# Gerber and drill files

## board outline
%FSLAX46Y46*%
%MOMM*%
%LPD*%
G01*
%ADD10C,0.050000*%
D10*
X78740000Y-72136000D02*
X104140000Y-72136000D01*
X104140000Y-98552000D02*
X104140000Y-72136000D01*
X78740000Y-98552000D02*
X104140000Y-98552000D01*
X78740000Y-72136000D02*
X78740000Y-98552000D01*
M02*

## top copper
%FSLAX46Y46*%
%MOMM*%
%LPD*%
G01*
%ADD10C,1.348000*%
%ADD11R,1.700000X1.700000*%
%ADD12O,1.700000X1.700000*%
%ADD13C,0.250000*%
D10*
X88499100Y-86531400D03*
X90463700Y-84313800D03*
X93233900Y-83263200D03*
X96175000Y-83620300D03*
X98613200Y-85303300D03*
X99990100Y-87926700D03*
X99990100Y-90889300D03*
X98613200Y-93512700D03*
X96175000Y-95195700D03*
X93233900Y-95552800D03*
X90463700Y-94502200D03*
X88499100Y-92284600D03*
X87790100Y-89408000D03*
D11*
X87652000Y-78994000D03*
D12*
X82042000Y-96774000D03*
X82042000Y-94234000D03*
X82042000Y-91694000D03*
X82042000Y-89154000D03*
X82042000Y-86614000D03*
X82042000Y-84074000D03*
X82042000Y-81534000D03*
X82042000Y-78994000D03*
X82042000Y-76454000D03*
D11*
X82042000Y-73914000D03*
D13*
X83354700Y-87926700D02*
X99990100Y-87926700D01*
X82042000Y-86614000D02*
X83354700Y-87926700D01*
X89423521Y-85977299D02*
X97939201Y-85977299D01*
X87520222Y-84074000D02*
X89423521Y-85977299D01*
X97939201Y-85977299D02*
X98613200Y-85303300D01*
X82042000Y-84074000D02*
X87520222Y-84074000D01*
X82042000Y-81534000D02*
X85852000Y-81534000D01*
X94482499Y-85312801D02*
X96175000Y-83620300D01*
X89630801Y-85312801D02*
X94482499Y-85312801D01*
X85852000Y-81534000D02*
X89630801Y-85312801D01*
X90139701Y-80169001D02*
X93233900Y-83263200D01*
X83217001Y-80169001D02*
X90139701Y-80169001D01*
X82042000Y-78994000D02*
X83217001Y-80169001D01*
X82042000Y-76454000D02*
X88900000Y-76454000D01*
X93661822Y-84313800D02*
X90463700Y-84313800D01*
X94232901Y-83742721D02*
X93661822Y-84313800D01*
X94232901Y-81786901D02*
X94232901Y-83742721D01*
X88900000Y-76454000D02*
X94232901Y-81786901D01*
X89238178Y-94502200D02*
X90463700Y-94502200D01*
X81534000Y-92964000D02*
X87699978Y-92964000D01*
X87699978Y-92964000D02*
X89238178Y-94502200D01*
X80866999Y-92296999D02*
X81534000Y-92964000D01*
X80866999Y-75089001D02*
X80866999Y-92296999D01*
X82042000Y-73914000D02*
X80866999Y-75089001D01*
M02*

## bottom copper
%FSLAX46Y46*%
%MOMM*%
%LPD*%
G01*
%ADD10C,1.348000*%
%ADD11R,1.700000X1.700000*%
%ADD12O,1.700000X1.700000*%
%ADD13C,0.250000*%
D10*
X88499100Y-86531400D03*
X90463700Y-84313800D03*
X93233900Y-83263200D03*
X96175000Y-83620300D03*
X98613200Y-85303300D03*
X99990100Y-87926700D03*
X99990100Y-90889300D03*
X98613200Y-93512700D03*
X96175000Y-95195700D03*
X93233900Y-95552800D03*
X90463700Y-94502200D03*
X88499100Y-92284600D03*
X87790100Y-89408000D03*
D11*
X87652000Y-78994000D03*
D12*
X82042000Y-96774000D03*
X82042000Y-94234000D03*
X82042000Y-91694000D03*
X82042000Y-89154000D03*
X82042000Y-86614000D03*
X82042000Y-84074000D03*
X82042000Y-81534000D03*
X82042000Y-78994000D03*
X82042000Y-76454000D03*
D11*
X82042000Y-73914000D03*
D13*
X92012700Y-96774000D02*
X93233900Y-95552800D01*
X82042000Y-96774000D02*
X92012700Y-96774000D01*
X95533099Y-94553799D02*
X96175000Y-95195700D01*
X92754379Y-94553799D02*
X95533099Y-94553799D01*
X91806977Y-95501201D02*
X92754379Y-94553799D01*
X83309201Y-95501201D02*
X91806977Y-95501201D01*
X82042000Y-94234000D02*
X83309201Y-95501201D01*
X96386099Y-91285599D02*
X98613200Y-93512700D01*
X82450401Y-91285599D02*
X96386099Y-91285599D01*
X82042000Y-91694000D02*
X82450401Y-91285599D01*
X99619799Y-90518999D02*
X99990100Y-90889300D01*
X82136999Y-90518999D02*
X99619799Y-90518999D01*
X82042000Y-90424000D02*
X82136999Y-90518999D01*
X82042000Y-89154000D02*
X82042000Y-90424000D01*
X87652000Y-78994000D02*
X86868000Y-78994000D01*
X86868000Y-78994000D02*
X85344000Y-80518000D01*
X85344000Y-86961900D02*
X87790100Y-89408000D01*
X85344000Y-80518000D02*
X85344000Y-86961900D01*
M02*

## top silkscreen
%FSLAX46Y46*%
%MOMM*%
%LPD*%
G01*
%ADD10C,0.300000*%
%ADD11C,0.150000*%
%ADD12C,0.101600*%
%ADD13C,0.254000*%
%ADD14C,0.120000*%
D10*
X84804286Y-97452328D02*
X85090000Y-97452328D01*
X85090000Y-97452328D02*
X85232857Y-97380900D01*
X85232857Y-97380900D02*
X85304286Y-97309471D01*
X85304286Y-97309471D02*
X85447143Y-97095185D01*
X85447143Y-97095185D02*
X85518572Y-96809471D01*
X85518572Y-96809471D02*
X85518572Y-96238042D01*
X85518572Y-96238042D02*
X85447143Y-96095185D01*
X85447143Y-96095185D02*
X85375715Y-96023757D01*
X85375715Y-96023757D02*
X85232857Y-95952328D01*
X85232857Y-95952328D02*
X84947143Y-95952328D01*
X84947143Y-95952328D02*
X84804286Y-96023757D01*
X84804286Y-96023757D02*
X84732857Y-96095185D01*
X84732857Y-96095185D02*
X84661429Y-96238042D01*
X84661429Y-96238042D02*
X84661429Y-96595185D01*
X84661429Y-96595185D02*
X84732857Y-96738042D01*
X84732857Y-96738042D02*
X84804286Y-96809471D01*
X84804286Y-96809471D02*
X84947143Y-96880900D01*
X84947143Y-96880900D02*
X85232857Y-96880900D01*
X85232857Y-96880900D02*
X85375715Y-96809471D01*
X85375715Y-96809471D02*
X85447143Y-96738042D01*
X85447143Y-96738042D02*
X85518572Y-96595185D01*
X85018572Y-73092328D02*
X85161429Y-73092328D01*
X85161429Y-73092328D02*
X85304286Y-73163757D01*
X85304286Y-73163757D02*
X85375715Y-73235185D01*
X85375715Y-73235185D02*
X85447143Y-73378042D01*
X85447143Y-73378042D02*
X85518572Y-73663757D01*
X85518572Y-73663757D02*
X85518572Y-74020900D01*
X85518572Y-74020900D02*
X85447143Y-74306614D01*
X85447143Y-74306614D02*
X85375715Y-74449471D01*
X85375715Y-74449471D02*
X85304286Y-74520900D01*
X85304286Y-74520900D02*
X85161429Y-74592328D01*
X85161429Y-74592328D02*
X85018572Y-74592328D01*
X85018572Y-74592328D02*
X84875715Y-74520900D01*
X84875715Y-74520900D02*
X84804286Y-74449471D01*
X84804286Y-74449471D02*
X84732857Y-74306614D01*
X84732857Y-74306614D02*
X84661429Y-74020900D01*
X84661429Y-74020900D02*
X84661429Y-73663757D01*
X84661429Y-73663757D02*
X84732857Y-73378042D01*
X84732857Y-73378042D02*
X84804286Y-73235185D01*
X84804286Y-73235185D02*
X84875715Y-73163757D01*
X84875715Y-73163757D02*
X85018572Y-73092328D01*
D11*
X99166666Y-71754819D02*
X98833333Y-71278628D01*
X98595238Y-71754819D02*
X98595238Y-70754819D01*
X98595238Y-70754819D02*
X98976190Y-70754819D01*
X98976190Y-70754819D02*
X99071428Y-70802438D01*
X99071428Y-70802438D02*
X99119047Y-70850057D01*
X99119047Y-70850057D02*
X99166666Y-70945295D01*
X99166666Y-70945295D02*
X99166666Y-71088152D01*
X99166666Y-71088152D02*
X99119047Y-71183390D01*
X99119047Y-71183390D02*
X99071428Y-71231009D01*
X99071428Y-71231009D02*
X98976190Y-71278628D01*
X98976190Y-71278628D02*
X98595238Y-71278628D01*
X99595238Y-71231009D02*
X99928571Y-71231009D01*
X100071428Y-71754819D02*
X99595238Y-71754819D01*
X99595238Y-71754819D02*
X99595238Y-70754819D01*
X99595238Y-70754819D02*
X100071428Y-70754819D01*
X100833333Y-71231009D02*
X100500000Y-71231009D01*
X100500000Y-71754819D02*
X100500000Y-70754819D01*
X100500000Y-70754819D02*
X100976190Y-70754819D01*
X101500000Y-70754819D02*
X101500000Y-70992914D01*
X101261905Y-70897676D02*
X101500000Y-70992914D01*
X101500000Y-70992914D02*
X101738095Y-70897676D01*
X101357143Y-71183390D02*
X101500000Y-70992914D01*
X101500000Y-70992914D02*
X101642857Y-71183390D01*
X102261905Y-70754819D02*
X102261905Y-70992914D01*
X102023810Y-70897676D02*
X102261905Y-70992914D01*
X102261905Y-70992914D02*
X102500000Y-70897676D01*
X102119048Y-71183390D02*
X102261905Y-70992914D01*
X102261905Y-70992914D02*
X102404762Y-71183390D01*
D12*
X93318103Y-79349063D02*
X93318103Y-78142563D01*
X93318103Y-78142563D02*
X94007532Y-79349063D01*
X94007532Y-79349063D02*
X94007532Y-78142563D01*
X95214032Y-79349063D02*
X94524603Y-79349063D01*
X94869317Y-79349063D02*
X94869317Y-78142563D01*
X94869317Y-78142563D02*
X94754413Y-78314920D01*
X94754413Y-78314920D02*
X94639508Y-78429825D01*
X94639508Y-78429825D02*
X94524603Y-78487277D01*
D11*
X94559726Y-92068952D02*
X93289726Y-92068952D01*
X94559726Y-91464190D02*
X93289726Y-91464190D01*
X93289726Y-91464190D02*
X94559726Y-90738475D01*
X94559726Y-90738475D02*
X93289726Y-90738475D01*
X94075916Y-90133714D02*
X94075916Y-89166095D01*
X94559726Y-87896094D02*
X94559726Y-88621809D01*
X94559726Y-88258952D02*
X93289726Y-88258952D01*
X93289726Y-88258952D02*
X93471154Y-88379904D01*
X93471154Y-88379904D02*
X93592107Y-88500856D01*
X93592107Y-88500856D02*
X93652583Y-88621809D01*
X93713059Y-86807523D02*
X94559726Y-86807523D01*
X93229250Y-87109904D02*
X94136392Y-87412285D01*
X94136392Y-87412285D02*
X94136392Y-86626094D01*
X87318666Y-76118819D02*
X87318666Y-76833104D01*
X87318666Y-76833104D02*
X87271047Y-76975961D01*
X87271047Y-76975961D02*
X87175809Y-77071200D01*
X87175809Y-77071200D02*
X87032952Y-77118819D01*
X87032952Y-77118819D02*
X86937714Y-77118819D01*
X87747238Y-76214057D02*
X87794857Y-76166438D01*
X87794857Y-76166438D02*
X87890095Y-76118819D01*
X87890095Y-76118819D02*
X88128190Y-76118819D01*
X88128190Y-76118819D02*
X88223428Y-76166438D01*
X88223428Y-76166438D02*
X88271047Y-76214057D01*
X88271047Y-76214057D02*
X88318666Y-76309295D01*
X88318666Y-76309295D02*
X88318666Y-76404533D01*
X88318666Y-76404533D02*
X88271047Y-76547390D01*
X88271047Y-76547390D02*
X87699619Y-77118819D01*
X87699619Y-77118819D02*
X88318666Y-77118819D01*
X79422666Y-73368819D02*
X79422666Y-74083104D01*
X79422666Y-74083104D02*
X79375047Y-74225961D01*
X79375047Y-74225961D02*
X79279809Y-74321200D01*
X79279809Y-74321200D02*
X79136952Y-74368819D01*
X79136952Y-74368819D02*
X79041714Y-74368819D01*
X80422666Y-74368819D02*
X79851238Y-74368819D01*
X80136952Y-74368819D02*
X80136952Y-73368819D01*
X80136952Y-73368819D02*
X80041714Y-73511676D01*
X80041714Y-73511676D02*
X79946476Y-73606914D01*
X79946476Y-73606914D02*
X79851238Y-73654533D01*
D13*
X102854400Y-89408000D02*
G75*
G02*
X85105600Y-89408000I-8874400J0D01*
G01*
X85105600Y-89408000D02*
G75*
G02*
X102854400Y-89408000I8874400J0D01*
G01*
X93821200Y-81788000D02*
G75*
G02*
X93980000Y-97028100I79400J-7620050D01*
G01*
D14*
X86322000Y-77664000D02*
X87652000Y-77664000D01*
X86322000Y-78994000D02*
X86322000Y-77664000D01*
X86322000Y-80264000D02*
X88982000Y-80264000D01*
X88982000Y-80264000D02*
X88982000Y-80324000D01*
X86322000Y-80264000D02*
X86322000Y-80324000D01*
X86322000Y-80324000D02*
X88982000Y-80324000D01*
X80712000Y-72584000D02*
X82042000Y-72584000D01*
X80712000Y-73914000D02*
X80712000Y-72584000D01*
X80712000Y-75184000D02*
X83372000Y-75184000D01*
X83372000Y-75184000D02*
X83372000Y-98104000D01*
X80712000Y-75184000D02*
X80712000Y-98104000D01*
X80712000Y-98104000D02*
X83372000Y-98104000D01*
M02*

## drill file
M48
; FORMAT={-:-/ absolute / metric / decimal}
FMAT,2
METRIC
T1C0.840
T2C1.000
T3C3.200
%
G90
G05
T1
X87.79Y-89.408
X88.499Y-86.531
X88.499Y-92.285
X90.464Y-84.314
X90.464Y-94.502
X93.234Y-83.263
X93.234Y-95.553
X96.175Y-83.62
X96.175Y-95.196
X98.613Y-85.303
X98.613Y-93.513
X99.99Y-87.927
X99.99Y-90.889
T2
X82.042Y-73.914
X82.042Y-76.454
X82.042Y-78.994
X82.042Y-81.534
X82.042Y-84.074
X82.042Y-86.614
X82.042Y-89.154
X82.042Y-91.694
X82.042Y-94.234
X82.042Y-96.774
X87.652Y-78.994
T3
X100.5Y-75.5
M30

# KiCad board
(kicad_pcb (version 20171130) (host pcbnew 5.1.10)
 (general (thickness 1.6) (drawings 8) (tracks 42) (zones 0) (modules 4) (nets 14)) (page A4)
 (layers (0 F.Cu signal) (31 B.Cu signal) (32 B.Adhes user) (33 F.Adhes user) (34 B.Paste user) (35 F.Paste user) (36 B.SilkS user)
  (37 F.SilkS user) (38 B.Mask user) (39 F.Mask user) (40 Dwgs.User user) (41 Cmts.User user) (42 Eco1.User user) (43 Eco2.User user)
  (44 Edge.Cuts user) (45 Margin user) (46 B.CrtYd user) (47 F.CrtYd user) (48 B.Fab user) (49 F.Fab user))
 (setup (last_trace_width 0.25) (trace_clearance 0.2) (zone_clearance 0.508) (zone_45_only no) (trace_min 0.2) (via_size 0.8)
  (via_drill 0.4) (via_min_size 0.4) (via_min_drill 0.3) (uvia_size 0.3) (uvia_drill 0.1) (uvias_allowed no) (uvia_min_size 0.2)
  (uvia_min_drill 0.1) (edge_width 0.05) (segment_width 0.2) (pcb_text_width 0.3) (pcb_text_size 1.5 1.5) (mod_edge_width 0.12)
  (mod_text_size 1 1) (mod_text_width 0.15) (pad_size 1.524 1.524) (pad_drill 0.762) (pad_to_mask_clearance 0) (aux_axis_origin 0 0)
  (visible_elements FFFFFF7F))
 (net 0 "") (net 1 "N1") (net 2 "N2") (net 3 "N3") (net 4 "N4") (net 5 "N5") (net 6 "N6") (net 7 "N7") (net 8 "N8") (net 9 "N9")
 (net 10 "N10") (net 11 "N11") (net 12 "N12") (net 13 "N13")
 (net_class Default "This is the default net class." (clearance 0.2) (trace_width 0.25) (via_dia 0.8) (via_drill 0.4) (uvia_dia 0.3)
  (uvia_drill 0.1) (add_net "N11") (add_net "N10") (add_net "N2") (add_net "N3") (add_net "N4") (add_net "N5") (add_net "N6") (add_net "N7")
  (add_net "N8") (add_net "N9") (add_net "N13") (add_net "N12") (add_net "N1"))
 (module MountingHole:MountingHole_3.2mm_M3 (layer F.Cu) (at 100.5 75.5)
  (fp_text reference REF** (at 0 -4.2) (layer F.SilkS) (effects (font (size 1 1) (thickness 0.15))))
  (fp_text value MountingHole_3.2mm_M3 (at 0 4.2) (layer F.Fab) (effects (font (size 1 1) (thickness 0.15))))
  (pad 1 np_thru_hole circle (at 0 0) (size 3.2 3.2) (drill 3.2) (layers *.Cu *.Mask)))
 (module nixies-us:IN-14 (layer F.Cu) (at 93.98 89.408 270)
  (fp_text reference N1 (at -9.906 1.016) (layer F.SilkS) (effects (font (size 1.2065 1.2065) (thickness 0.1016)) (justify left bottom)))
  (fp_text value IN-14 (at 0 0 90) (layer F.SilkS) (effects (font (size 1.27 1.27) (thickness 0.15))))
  (fp_circle (center 0 0) (end 8.8744 0) (layer F.SilkS) (width 0.254))
  (fp_arc (start 0.00005 0.0794) (end -7.62 0.1588) (angle 180) (layer F.SilkS) (width 0.254))
  (pad RHDP thru_hole circle (at -2.8766 5.4809 270) (size 1.348 1.348) (drill 0.84) (layers *.Cu *.Mask) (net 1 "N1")
   (solder_mask_margin 0.1016))
  (pad 1 thru_hole circle (at -5.0942 3.5163 270) (size 1.348 1.348) (drill 0.84) (layers *.Cu *.Mask) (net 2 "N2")
   (solder_mask_margin 0.1016))
  (pad 2 thru_hole circle (at -6.1448 0.7461 270) (size 1.348 1.348) (drill 0.84) (layers *.Cu *.Mask) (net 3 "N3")
   (solder_mask_margin 0.1016))
  (pad 3 thru_hole circle (at -5.7877 -2.195 270) (size 1.348 1.348) (drill 0.84) (layers *.Cu *.Mask) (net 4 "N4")
   (solder_mask_margin 0.1016))
  (pad 4 thru_hole circle (at -4.1047 -4.6332 270) (size 1.348 1.348) (drill 0.84) (layers *.Cu *.Mask) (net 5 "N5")
   (solder_mask_margin 0.1016))
  (pad 5 thru_hole circle (at -1.4813 -6.0101 270) (size 1.348 1.348) (drill 0.84) (layers *.Cu *.Mask) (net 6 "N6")
   (solder_mask_margin 0.1016))
  (pad 6 thru_hole circle (at 1.4813 -6.0101 270) (size 1.348 1.348) (drill 0.84) (layers *.Cu *.Mask) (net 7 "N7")
   (solder_mask_margin 0.1016))
  (pad 7 thru_hole circle (at 4.1047 -4.6332 270) (size 1.348 1.348) (drill 0.84) (layers *.Cu *.Mask) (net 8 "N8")
   (solder_mask_margin 0.1016))
  (pad 8 thru_hole circle (at 5.7877 -2.195 270) (size 1.348 1.348) (drill 0.84) (layers *.Cu *.Mask) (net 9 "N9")
   (solder_mask_margin 0.1016))
  (pad 9 thru_hole circle (at 6.1448 0.7461 270) (size 1.348 1.348) (drill 0.84) (layers *.Cu *.Mask) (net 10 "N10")
   (solder_mask_margin 0.1016))
  (pad 0 thru_hole circle (at 5.0942 3.5163 270) (size 1.348 1.348) (drill 0.84) (layers *.Cu *.Mask) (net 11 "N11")
   (solder_mask_margin 0.1016))
  (pad LHDP thru_hole circle (at 2.8766 5.4809 270) (size 1.348 1.348) (drill 0.84) (layers *.Cu *.Mask) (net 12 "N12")
   (solder_mask_margin 0.1016))
  (pad A thru_hole circle (at 0 6.1899 270) (size 1.348 1.348) (drill 0.84) (layers *.Cu *.Mask) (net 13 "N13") (solder_mask_margin 0.1016)))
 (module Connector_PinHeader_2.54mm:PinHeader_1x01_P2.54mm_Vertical (layer F.Cu) (at 87.652 78.994)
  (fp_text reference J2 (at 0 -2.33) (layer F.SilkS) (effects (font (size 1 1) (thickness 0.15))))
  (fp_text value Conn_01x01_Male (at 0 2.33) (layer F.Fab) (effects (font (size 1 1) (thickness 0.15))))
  (fp_line (start -1.33 -1.33) (end 0 -1.33) (layer F.SilkS) (width 0.12))
  (fp_line (start -1.33 0) (end -1.33 -1.33) (layer F.SilkS) (width 0.12))
  (fp_line (start -1.33 1.27) (end 1.33 1.27) (layer F.SilkS) (width 0.12))
  (fp_line (start 1.33 1.27) (end 1.33 1.33) (layer F.SilkS) (width 0.12))
  (fp_line (start -1.33 1.27) (end -1.33 1.33) (layer F.SilkS) (width 0.12))
  (fp_line (start -1.33 1.33) (end 1.33 1.33) (layer F.SilkS) (width 0.12))
  (pad 1 thru_hole rect (at 0 0) (size 1.7 1.7) (drill 1) (layers *.Cu *.Mask) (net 13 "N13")))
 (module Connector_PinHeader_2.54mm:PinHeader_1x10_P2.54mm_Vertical (layer F.Cu) (at 82.042 73.914)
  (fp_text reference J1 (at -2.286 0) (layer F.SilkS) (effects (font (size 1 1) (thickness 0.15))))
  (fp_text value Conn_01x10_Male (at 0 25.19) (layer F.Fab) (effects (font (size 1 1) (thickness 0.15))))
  (fp_line (start -1.33 -1.33) (end 0 -1.33) (layer F.SilkS) (width 0.12))
  (fp_line (start -1.33 0) (end -1.33 -1.33) (layer F.SilkS) (width 0.12))
  (fp_line (start -1.33 1.27) (end 1.33 1.27) (layer F.SilkS) (width 0.12))
  (fp_line (start 1.33 1.27) (end 1.33 24.19) (layer F.SilkS) (width 0.12))
  (fp_line (start -1.33 1.27) (end -1.33 24.19) (layer F.SilkS) (width 0.12))
  (fp_line (start -1.33 24.19) (end 1.33 24.19) (layer F.SilkS) (width 0.12))
  (pad 10 thru_hole oval (at 0 22.86) (size 1.7 1.7) (drill 1) (layers *.Cu *.Mask) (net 10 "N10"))
  (pad 9 thru_hole oval (at 0 20.32) (size 1.7 1.7) (drill 1) (layers *.Cu *.Mask) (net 9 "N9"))
  (pad 8 thru_hole oval (at 0 17.78) (size 1.7 1.7) (drill 1) (layers *.Cu *.Mask) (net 8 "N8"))
  (pad 7 thru_hole oval (at 0 15.24) (size 1.7 1.7) (drill 1) (layers *.Cu *.Mask) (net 7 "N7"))
  (pad 6 thru_hole oval (at 0 12.7) (size 1.7 1.7) (drill 1) (layers *.Cu *.Mask) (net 6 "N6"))
  (pad 5 thru_hole oval (at 0 10.16) (size 1.7 1.7) (drill 1) (layers *.Cu *.Mask) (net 5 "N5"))
  (pad 4 thru_hole oval (at 0 7.62) (size 1.7 1.7) (drill 1) (layers *.Cu *.Mask) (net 4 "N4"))
  (pad 3 thru_hole oval (at 0 5.08) (size 1.7 1.7) (drill 1) (layers *.Cu *.Mask) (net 3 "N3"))
  (pad 2 thru_hole oval (at 0 2.54) (size 1.7 1.7) (drill 1) (layers *.Cu *.Mask) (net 2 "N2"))
  (pad 1 thru_hole rect (at 0 0) (size 1.7 1.7) (drill 1) (layers *.Cu *.Mask) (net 11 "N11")))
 (gr_line (start 78.74 72.136) (end 104.14 72.136) (layer Edge.Cuts) (width 0.05))
 (gr_line (start 104.14 98.552) (end 104.14 72.136) (layer Edge.Cuts) (width 0.05))
 (gr_line (start 78.74 98.552) (end 104.14 98.552) (layer Edge.Cuts) (width 0.05))
 (gr_line (start 78.74 72.136) (end 78.74 98.552) (layer Edge.Cuts) (width 0.05))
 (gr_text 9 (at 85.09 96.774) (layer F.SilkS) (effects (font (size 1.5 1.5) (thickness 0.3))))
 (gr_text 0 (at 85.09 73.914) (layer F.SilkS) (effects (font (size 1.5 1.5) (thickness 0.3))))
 (segment (start 92.0127 96.774) (end 93.2339 95.5528) (width 0.25) (layer B.Cu) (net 10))
 (segment (start 82.042 96.774) (end 92.0127 96.774) (width 0.25) (layer B.Cu) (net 10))
 (segment (start 95.533099 94.553799) (end 96.175 95.1957) (width 0.25) (layer B.Cu) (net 9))
 (segment (start 92.754379 94.553799) (end 95.533099 94.553799) (width 0.25) (layer B.Cu) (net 9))
 (segment (start 91.806977 95.501201) (end 92.754379 94.553799) (width 0.25) (layer B.Cu) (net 9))
 (segment (start 83.309201 95.501201) (end 91.806977 95.501201) (width 0.25) (layer B.Cu) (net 9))
 (segment (start 82.042 94.234) (end 83.309201 95.501201) (width 0.25) (layer B.Cu) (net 9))
 (segment (start 96.386099 91.285599) (end 98.6132 93.5127) (width 0.25) (layer B.Cu) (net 8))
 (segment (start 82.450401 91.285599) (end 96.386099 91.285599) (width 0.25) (layer B.Cu) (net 8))
 (segment (start 82.042 91.694) (end 82.450401 91.285599) (width 0.25) (layer B.Cu) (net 8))
 (segment (start 99.619799 90.518999) (end 99.9901 90.8893) (width 0.25) (layer B.Cu) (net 7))
 (segment (start 82.136999 90.518999) (end 99.619799 90.518999) (width 0.25) (layer B.Cu) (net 7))
 (segment (start 82.042 90.424) (end 82.136999 90.518999) (width 0.25) (layer B.Cu) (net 7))
 (segment (start 82.042 89.154) (end 82.042 90.424) (width 0.25) (layer B.Cu) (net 7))
 (segment (start 83.3547 87.9267) (end 99.9901 87.9267) (width 0.25) (layer F.Cu) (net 6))
 (segment (start 82.042 86.614) (end 83.3547 87.9267) (width 0.25) (layer F.Cu) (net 6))
 (segment (start 89.423521 85.977299) (end 97.939201 85.977299) (width 0.25) (layer F.Cu) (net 5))
 (segment (start 87.520222 84.074) (end 89.423521 85.977299) (width 0.25) (layer F.Cu) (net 5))
 (segment (start 97.939201 85.977299) (end 98.6132 85.3033) (width 0.25) (layer F.Cu) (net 5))
 (segment (start 82.042 84.074) (end 87.520222 84.074) (width 0.25) (layer F.Cu) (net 5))
 (segment (start 82.042 81.534) (end 85.852 81.534) (width 0.25) (layer F.Cu) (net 4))
 (segment (start 94.482499 85.312801) (end 96.175 83.6203) (width 0.25) (layer F.Cu) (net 4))
 (segment (start 89.630801 85.312801) (end 94.482499 85.312801) (width 0.25) (layer F.Cu) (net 4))
 (segment (start 85.852 81.534) (end 89.630801 85.312801) (width 0.25) (layer F.Cu) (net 4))
 (segment (start 90.139701 80.169001) (end 93.2339 83.2632) (width 0.25) (layer F.Cu) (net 3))
 (segment (start 83.217001 80.169001) (end 90.139701 80.169001) (width 0.25) (layer F.Cu) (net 3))
 (segment (start 82.042 78.994) (end 83.217001 80.169001) (width 0.25) (layer F.Cu) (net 3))
 (segment (start 82.042 76.454) (end 88.9 76.454) (width 0.25) (layer F.Cu) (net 2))
 (segment (start 93.661822 84.3138) (end 90.4637 84.3138) (width 0.25) (layer F.Cu) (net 2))
 (segment (start 94.232901 83.742721) (end 93.661822 84.3138) (width 0.25) (layer F.Cu) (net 2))
 (segment (start 94.232901 81.786901) (end 94.232901 83.742721) (width 0.25) (layer F.Cu) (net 2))
 (segment (start 88.9 76.454) (end 94.232901 81.786901) (width 0.25) (layer F.Cu) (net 2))
 (segment (start 89.238178 94.5022) (end 90.4637 94.5022) (width 0.25) (layer F.Cu) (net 11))
 (segment (start 81.534 92.964) (end 87.699978 92.964) (width 0.25) (layer F.Cu) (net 11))
 (segment (start 87.699978 92.964) (end 89.238178 94.5022) (width 0.25) (layer F.Cu) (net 11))
 (segment (start 80.866999 92.296999) (end 81.534 92.964) (width 0.25) (layer F.Cu) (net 11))
 (segment (start 80.866999 75.089001) (end 80.866999 92.296999) (width 0.25) (layer F.Cu) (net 11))
 (segment (start 82.042 73.914) (end 80.866999 75.089001) (width 0.25) (layer F.Cu) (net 11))
 (segment (start 87.652 78.994) (end 86.868 78.994) (width 0.25) (layer B.Cu) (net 13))
 (segment (start 86.868 78.994) (end 85.344 80.518) (width 0.25) (layer B.Cu) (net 13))
 (segment (start 85.344 86.9619) (end 87.7901 89.408) (width 0.25) (layer B.Cu) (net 13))
 (segment (start 85.344 80.518) (end 85.344 86.9619) (width 0.25) (layer B.Cu) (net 13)))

